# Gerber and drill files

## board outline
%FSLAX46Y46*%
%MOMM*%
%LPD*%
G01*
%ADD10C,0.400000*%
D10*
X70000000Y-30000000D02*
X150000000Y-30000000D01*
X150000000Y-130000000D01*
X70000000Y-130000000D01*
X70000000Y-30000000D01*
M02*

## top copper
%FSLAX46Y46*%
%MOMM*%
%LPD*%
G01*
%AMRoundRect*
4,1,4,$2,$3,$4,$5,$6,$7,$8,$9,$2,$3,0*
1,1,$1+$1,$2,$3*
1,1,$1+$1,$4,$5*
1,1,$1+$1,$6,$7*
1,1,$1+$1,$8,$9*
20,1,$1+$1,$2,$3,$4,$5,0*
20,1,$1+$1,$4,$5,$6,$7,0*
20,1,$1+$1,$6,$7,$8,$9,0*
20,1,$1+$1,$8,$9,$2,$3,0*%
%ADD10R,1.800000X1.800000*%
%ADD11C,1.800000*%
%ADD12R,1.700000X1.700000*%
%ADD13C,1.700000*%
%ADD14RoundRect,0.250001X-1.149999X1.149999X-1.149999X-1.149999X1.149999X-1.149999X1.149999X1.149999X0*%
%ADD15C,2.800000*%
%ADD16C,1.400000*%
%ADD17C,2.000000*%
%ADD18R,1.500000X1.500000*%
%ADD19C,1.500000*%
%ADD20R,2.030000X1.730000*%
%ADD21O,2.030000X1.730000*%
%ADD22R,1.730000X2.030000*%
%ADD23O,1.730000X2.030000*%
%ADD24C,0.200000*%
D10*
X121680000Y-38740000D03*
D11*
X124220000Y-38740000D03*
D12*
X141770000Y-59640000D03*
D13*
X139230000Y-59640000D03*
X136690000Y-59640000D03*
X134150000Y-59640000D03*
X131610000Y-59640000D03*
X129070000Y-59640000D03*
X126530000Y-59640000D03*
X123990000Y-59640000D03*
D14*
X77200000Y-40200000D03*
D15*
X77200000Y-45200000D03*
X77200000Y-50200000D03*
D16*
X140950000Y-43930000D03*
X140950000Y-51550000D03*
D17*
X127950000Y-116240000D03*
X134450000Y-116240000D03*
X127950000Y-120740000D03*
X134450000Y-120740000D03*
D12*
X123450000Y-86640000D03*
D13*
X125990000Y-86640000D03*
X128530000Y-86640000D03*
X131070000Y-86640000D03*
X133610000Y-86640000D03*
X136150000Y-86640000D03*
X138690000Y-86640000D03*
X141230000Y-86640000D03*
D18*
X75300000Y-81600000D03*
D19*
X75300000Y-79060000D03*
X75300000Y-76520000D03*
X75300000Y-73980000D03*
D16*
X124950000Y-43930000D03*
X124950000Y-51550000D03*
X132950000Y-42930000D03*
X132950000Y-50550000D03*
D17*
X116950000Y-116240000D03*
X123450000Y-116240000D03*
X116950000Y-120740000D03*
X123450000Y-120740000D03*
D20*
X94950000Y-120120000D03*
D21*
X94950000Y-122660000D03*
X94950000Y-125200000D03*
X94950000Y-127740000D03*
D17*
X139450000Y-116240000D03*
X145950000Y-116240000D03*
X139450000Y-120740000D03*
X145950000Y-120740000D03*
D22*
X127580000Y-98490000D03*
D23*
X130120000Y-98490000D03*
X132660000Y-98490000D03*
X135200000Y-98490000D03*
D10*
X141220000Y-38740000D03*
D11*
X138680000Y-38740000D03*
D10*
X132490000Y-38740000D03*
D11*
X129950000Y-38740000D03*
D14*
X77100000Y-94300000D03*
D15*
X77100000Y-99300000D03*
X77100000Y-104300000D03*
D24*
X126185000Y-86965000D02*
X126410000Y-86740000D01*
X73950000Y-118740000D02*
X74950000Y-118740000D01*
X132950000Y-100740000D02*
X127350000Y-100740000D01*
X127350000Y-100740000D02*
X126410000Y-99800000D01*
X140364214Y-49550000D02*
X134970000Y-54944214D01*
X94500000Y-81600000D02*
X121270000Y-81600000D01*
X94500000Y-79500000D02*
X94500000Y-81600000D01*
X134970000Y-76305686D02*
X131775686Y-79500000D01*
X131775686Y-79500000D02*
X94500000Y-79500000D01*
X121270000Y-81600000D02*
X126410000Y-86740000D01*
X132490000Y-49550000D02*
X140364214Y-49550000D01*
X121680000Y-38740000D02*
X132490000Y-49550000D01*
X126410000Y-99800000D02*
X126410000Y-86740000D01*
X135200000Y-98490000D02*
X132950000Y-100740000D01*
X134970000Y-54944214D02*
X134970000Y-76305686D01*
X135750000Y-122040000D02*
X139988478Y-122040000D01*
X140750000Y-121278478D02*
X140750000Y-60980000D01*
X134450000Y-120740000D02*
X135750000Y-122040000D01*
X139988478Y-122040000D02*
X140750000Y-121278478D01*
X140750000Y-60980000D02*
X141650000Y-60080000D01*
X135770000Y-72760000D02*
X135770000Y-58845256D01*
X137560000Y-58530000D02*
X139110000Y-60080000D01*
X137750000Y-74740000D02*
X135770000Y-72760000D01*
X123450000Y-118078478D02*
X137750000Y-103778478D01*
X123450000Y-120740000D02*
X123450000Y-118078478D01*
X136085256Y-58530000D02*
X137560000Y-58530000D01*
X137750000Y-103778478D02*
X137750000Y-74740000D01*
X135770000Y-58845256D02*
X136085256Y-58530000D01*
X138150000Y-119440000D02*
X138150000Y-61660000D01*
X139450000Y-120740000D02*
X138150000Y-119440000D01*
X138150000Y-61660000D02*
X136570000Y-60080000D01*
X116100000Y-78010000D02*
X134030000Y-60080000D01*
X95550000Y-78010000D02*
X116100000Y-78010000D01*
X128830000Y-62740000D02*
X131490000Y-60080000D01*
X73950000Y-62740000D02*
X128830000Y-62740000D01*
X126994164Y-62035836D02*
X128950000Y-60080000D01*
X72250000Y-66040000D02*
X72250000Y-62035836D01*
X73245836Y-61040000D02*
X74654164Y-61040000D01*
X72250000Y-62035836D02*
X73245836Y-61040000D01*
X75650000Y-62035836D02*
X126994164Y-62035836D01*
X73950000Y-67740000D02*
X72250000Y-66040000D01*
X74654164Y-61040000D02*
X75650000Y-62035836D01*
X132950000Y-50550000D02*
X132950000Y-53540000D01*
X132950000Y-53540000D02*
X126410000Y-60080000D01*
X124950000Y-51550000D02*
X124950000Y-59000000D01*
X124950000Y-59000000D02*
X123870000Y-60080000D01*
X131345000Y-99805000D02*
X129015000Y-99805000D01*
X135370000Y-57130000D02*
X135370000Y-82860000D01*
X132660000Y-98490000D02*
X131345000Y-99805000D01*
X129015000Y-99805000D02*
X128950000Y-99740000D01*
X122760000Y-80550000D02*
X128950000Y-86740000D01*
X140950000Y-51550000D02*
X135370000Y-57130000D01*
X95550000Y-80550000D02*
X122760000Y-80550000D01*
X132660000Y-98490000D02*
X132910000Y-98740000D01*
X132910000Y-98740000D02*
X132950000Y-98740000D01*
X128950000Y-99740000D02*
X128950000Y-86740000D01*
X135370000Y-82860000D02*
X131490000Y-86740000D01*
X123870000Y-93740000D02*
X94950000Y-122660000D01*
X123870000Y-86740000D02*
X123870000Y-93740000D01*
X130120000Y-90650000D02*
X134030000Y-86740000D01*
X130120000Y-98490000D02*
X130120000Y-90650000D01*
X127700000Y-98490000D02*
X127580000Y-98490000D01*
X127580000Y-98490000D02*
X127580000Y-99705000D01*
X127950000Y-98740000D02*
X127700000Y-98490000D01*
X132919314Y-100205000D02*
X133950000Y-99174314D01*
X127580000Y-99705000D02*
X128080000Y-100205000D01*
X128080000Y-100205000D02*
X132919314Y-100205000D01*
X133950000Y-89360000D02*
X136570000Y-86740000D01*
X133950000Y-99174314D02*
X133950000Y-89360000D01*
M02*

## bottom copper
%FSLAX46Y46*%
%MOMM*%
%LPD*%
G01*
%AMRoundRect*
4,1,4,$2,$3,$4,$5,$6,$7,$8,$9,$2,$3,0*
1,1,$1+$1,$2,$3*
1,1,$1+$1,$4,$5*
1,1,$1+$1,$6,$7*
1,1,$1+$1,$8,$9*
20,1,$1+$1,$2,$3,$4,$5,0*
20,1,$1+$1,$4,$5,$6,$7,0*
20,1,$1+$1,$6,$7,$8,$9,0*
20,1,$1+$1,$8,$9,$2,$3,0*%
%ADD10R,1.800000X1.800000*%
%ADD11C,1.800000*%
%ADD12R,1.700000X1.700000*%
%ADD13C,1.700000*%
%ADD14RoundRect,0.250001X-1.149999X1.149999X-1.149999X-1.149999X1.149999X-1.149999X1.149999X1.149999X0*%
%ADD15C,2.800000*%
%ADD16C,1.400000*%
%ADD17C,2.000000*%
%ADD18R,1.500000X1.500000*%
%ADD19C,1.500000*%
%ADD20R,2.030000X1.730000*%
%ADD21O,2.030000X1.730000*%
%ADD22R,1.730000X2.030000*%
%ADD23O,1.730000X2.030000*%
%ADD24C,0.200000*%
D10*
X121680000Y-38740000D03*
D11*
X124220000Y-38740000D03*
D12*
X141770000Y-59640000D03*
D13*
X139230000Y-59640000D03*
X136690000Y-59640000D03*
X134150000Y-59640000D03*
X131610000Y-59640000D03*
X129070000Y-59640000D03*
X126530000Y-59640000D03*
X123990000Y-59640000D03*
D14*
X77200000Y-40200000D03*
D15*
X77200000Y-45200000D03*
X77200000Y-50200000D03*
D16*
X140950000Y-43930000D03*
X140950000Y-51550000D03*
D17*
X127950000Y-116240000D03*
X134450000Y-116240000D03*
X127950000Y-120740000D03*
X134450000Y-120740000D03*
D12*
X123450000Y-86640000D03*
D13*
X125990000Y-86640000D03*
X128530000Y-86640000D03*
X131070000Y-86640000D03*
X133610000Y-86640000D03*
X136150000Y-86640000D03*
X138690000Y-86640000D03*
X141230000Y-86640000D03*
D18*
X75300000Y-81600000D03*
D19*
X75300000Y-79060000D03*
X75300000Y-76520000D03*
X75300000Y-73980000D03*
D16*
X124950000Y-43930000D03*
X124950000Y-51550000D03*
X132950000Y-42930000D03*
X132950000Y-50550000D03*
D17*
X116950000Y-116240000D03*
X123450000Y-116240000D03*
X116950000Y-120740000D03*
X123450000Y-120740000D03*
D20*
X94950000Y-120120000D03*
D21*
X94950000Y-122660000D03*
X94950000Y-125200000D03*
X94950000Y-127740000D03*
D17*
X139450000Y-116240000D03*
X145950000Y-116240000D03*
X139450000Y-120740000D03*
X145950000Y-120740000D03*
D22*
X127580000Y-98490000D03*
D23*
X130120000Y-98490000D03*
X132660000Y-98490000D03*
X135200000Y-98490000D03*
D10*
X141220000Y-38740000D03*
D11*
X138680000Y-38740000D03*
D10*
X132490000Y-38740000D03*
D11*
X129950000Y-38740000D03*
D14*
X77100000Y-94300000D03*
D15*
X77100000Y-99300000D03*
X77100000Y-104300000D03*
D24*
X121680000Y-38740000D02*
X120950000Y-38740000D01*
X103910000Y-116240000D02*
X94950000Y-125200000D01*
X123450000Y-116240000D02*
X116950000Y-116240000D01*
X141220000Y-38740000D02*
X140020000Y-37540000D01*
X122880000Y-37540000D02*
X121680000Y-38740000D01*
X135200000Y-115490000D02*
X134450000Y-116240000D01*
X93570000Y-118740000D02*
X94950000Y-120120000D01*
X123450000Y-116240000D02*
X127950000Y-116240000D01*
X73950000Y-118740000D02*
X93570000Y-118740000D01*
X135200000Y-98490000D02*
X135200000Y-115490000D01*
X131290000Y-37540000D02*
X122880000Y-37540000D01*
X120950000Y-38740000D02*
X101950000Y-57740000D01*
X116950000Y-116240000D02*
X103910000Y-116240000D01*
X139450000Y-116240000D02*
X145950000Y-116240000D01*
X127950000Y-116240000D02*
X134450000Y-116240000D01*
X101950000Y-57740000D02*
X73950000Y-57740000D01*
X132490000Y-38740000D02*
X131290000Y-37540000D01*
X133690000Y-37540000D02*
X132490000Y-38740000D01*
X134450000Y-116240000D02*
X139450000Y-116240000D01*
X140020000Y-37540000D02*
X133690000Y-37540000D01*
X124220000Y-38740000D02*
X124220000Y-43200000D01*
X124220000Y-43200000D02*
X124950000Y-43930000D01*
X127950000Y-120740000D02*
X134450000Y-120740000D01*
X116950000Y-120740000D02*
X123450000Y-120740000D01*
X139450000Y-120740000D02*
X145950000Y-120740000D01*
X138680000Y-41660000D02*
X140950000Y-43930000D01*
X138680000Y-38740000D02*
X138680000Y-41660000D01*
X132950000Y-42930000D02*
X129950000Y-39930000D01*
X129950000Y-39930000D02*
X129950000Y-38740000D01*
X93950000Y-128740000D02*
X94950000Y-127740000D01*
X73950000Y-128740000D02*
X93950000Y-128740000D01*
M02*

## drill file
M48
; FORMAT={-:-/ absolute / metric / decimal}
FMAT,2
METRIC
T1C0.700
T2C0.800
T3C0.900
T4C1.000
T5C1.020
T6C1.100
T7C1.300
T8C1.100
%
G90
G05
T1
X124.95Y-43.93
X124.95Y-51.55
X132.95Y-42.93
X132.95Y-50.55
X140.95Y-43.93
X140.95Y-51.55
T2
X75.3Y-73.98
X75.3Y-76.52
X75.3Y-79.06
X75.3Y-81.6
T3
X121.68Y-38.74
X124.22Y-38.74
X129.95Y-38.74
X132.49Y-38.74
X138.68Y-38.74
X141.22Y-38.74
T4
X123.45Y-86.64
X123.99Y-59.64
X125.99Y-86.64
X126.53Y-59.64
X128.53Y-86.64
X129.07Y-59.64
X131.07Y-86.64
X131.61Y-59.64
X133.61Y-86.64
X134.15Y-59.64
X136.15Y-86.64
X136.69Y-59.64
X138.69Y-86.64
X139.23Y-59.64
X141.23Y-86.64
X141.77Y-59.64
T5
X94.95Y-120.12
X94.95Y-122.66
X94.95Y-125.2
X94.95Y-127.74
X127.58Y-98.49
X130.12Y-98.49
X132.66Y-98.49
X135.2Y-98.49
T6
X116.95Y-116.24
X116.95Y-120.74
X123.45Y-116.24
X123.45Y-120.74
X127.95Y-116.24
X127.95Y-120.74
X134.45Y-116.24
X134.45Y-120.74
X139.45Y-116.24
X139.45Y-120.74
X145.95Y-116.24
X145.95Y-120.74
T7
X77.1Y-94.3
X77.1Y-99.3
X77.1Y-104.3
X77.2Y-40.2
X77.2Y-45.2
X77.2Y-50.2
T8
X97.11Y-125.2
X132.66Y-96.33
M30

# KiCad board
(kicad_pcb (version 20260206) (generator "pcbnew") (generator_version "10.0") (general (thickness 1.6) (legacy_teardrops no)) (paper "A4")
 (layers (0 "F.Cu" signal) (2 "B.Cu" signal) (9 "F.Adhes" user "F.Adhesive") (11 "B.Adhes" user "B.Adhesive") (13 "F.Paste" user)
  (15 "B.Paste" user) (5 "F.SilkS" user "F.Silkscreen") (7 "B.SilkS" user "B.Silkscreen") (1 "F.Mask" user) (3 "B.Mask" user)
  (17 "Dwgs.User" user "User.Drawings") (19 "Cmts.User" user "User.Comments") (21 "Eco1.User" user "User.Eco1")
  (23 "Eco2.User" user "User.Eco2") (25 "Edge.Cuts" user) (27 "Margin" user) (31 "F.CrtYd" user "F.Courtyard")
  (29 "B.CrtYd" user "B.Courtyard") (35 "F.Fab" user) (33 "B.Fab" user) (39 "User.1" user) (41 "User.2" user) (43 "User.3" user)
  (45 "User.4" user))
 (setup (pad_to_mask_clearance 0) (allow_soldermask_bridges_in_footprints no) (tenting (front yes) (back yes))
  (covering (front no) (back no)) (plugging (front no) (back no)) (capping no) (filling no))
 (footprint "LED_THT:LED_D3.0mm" (layer "F.Cu") (at 121.68 38.74)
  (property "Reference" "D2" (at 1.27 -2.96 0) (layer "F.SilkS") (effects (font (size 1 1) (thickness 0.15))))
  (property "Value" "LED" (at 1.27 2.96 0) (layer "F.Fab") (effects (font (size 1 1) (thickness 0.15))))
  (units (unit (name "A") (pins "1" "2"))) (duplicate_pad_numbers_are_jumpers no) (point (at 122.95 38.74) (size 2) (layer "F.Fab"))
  (pad "1" thru_hole rect (at 0 0) (size 1.8 1.8) (drill 0.9) (layers "*.Cu" "*.Mask") (remove_unused_layers no) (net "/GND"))
  (pad "2" thru_hole circle (at 2.54 0) (size 1.8 1.8) (drill 0.9) (layers "*.Cu" "*.Mask") (remove_unused_layers no) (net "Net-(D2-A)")))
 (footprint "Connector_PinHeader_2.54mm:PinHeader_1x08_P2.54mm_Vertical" (layer "F.Cu") (at 141.77 59.64 -90)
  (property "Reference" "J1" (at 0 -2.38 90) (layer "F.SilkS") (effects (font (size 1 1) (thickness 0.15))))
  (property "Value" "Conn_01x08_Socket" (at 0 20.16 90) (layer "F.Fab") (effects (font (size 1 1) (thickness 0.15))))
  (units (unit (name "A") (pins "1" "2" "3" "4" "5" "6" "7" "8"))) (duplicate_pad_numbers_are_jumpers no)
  (pad "1" thru_hole rect (at 0 0 270) (size 1.7 1.7) (drill 1) (layers "*.Cu" "*.Mask") (remove_unused_layers no) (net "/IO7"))
  (pad "2" thru_hole circle (at 0 2.54 270) (size 1.7 1.7) (drill 1) (layers "*.Cu" "*.Mask") (remove_unused_layers no) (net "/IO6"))
  (pad "3" thru_hole circle (at 0 5.08 270) (size 1.7 1.7) (drill 1) (layers "*.Cu" "*.Mask") (remove_unused_layers no) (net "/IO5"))
  (pad "4" thru_hole circle (at 0 7.62 270) (size 1.7 1.7) (drill 1) (layers "*.Cu" "*.Mask") (remove_unused_layers no) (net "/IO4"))
  (pad "5" thru_hole circle (at 0 10.16 270) (size 1.7 1.7) (drill 1) (layers "*.Cu" "*.Mask") (remove_unused_layers no) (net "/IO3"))
  (pad "6" thru_hole circle (at 0 12.7 270) (size 1.7 1.7) (drill 1) (layers "*.Cu" "*.Mask") (remove_unused_layers no) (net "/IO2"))
  (pad "7" thru_hole circle (at 0 15.24 270) (size 1.7 1.7) (drill 1) (layers "*.Cu" "*.Mask") (remove_unused_layers no) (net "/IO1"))
  (pad "8" thru_hole circle (at 0 17.78 270) (size 1.7 1.7) (drill 1) (layers "*.Cu" "*.Mask") (remove_unused_layers no) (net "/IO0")))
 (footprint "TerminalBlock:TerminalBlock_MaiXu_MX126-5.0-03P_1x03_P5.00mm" (layer "F.Cu") (at 77.2 40.2 -90)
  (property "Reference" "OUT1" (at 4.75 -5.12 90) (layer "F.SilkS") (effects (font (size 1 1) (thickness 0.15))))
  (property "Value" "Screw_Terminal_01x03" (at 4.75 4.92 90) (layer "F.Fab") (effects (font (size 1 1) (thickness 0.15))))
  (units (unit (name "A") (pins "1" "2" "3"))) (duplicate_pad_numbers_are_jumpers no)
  (pad "1" thru_hole roundrect (at 0 0 270) (size 2.8 2.8) (drill 1.3) (layers "*.Cu" "*.Mask") (remove_unused_layers no)
   (roundrect_rratio 0.089286) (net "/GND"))
  (pad "2" thru_hole circle (at 5 0 270) (size 2.8 2.8) (drill 1.3) (layers "*.Cu" "*.Mask") (remove_unused_layers no) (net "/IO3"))
  (pad "3" thru_hole circle (at 10 0 270) (size 2.8 2.8) (drill 1.3) (layers "*.Cu" "*.Mask") (remove_unused_layers no) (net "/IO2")))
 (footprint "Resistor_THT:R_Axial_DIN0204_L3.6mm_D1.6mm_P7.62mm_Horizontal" (layer "F.Cu") (at 140.95 43.93 -90)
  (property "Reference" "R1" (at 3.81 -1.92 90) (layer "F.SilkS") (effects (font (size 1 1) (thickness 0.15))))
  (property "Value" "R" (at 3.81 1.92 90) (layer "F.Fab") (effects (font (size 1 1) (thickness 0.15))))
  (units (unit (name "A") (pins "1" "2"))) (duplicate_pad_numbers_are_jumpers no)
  (pad "1" thru_hole circle (at 0 0 270) (size 1.4 1.4) (drill 0.7) (layers "*.Cu" "*.Mask") (remove_unused_layers no) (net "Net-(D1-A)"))
  (pad "2" thru_hole circle (at 7.62 0 270) (size 1.4 1.4) (drill 0.7) (layers "*.Cu" "*.Mask") (remove_unused_layers no) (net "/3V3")))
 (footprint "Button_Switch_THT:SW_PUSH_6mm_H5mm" (layer "F.Cu") (at 127.95 116.24)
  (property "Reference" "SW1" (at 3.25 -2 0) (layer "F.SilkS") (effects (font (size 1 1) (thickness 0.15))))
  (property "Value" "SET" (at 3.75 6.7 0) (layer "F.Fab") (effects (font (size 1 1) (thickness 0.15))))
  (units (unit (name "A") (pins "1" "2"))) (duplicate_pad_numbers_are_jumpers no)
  (pad "1" thru_hole circle (at 0 0 90) (size 2 2) (drill 1.1) (layers "*.Cu" "*.Mask") (remove_unused_layers no) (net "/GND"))
  (pad "1" thru_hole circle (at 6.5 0 90) (size 2 2) (drill 1.1) (layers "*.Cu" "*.Mask") (remove_unused_layers no) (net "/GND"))
  (pad "2" thru_hole circle (at 0 4.5 90) (size 2 2) (drill 1.1) (layers "*.Cu" "*.Mask") (remove_unused_layers no) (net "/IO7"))
  (pad "2" thru_hole circle (at 6.5 4.5 90) (size 2 2) (drill 1.1) (layers "*.Cu" "*.Mask") (remove_unused_layers no) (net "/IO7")))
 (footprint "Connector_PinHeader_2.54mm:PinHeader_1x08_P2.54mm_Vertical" (layer "F.Cu") (at 123.45 86.64 90)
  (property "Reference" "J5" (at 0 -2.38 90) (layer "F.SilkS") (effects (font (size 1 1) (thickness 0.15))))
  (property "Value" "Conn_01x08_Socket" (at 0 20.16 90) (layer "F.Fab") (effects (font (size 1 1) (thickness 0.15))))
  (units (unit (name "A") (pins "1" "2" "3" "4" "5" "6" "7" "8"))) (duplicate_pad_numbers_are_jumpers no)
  (pad "1" thru_hole rect (at 0 0 90) (size 1.7 1.7) (drill 1) (layers "*.Cu" "*.Mask") (remove_unused_layers no) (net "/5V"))
  (pad "2" thru_hole circle (at 0 2.54 90) (size 1.7 1.7) (drill 1) (layers "*.Cu" "*.Mask") (remove_unused_layers no) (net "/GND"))
  (pad "3" thru_hole circle (at 0 5.08 90) (size 1.7 1.7) (drill 1) (layers "*.Cu" "*.Mask") (remove_unused_layers no) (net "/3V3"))
  (pad "4" thru_hole circle (at 0 7.62 90) (size 1.7 1.7) (drill 1) (layers "*.Cu" "*.Mask") (remove_unused_layers no) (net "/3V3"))
  (pad "5" thru_hole circle (at 0 10.16 90) (size 1.7 1.7) (drill 1) (layers "*.Cu" "*.Mask") (remove_unused_layers no) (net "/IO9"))
  (pad "6" thru_hole circle (at 0 12.7 90) (size 1.7 1.7) (drill 1) (layers "*.Cu" "*.Mask") (remove_unused_layers no) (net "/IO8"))
  (pad "7" thru_hole circle (at 0 15.24 90) (size 1.7 1.7) (drill 1) (layers "*.Cu" "*.Mask") (remove_unused_layers no) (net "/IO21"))
  (pad "8" thru_hole circle (at 0 17.78 90) (size 1.7 1.7) (drill 1) (layers "*.Cu" "*.Mask") (remove_unused_layers no) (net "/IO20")))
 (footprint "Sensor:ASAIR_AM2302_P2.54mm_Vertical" (layer "F.Cu") (at 75.3 81.6 90)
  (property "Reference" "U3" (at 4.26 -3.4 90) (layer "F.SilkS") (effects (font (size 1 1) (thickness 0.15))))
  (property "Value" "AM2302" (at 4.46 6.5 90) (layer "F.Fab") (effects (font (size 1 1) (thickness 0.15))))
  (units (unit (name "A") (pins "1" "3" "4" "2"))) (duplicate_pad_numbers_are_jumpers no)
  (pad "1" thru_hole rect (at 0 0 180) (size 1.5 1.5) (drill 0.8) (layers "*.Cu" "*.Mask") (remove_unused_layers no) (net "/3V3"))
  (pad "2" thru_hole circle (at 2.54 0 180) (size 1.5 1.5) (drill 0.8) (layers "*.Cu" "*.Mask") (remove_unused_layers no) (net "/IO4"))
  (pad "3" thru_hole circle (at 5.08 0 180) (size 1.5 1.5) (drill 0.8) (layers "*.Cu" "*.Mask") (remove_unused_layers no)
   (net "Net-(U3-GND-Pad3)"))
  (pad "4" thru_hole circle (at 7.62 0 180) (size 1.5 1.5) (drill 0.8) (layers "*.Cu" "*.Mask") (remove_unused_layers no)
   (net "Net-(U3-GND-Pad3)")))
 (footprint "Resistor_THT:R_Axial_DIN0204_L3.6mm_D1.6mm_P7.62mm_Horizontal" (layer "F.Cu") (at 124.95 43.93 -90)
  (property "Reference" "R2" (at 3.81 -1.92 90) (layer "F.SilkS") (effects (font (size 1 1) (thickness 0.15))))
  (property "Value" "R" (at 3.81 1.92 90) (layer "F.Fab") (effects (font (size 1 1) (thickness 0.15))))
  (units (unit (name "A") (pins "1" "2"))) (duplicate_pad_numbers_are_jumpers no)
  (pad "1" thru_hole circle (at 0 0 270) (size 1.4 1.4) (drill 0.7) (layers "*.Cu" "*.Mask") (remove_unused_layers no) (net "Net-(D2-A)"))
  (pad "2" thru_hole circle (at 7.62 0 270) (size 1.4 1.4) (drill 0.7) (layers "*.Cu" "*.Mask") (remove_unused_layers no) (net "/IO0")))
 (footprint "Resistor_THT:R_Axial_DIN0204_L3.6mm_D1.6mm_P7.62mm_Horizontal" (layer "F.Cu") (at 132.95 42.93 -90)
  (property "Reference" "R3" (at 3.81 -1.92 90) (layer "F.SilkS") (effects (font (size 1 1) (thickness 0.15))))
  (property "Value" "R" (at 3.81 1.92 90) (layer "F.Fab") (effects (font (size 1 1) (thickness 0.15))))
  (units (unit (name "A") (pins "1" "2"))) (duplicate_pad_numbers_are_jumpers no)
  (pad "1" thru_hole circle (at 0 0 270) (size 1.4 1.4) (drill 0.7) (layers "*.Cu" "*.Mask") (remove_unused_layers no) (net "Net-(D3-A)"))
  (pad "2" thru_hole circle (at 7.62 0 270) (size 1.4 1.4) (drill 0.7) (layers "*.Cu" "*.Mask") (remove_unused_layers no) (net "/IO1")))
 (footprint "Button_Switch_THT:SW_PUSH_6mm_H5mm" (layer "F.Cu") (at 116.95 116.24)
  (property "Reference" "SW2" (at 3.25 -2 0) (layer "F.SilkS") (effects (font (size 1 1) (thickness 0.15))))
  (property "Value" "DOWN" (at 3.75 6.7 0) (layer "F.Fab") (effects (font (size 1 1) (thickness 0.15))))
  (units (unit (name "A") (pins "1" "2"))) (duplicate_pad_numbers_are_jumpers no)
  (pad "1" thru_hole circle (at 0 0 90) (size 2 2) (drill 1.1) (layers "*.Cu" "*.Mask") (remove_unused_layers no) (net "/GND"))
  (pad "1" thru_hole circle (at 6.5 0 90) (size 2 2) (drill 1.1) (layers "*.Cu" "*.Mask") (remove_unused_layers no) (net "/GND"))
  (pad "2" thru_hole circle (at 0 4.5 90) (size 2 2) (drill 1.1) (layers "*.Cu" "*.Mask") (remove_unused_layers no) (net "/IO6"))
  (pad "2" thru_hole circle (at 6.5 4.5 90) (size 2 2) (drill 1.1) (layers "*.Cu" "*.Mask") (remove_unused_layers no) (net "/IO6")))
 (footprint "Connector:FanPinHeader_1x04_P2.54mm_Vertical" (layer "F.Cu") (at 94.95 120.12 -90)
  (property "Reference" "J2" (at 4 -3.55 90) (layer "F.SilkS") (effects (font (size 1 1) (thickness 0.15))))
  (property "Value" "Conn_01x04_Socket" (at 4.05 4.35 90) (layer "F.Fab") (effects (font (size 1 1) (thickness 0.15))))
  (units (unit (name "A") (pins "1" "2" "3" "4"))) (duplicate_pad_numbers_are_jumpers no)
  (pad "" np_thru_hole circle (at 5.08 -2.16) (size 1.1 1.1) (drill 1.1) (layers "*.Cu" "*.Mask"))
  (pad "1" thru_hole rect (at 0 0) (size 2.03 1.73) (drill 1.02) (layers "*.Cu" "*.Mask") (remove_unused_layers no) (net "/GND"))
  (pad "2" thru_hole oval (at 2.54 0) (size 2.03 1.73) (drill 1.02) (layers "*.Cu" "*.Mask") (remove_unused_layers no) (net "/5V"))
  (pad "3" thru_hole oval (at 5.08 0) (size 2.03 1.73) (drill 1.02) (layers "*.Cu" "*.Mask") (remove_unused_layers no) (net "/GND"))
  (pad "4" thru_hole oval (at 7.62 0) (size 2.03 1.73) (drill 1.02) (layers "*.Cu" "*.Mask") (remove_unused_layers no) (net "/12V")))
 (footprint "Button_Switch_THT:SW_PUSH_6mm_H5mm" (layer "F.Cu") (at 139.45 116.24)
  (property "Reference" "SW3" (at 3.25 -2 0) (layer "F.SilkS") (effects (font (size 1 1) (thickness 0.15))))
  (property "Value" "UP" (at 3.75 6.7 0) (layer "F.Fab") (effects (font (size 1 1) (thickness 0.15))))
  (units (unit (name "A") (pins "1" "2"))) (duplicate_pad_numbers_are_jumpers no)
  (pad "1" thru_hole circle (at 0 0 90) (size 2 2) (drill 1.1) (layers "*.Cu" "*.Mask") (remove_unused_layers no) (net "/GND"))
  (pad "1" thru_hole circle (at 6.5 0 90) (size 2 2) (drill 1.1) (layers "*.Cu" "*.Mask") (remove_unused_layers no) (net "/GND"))
  (pad "2" thru_hole circle (at 0 4.5 90) (size 2 2) (drill 1.1) (layers "*.Cu" "*.Mask") (remove_unused_layers no) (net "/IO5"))
  (pad "2" thru_hole circle (at 6.5 4.5 90) (size 2 2) (drill 1.1) (layers "*.Cu" "*.Mask") (remove_unused_layers no) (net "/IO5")))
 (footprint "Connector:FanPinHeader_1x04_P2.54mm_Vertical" (layer "F.Cu") (at 127.58 98.49)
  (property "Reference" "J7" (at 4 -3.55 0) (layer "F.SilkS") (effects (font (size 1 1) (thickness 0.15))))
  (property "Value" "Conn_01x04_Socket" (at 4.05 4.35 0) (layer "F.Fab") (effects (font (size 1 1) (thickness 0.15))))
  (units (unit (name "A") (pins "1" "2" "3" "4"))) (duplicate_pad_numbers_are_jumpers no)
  (pad "" np_thru_hole circle (at 5.08 -2.16 90) (size 1.1 1.1) (drill 1.1) (layers "*.Cu" "*.Mask"))
  (pad "1" thru_hole rect (at 0 0 90) (size 2.03 1.73) (drill 1.02) (layers "*.Cu" "*.Mask") (remove_unused_layers no) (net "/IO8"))
  (pad "2" thru_hole oval (at 2.54 0 90) (size 2.03 1.73) (drill 1.02) (layers "*.Cu" "*.Mask") (remove_unused_layers no) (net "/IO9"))
  (pad "3" thru_hole oval (at 5.08 0 90) (size 2.03 1.73) (drill 1.02) (layers "*.Cu" "*.Mask") (remove_unused_layers no) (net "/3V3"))
  (pad "4" thru_hole oval (at 7.62 0 90) (size 2.03 1.73) (drill 1.02) (layers "*.Cu" "*.Mask") (remove_unused_layers no) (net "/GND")))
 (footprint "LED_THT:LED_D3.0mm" (layer "F.Cu") (at 141.22 38.74 180)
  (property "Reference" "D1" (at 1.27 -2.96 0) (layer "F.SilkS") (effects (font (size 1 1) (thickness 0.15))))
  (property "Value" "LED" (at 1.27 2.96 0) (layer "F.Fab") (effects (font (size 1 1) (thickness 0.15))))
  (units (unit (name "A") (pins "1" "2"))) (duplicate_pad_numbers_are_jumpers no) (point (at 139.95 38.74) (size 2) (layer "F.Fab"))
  (pad "1" thru_hole rect (at 0 0 180) (size 1.8 1.8) (drill 0.9) (layers "*.Cu" "*.Mask") (remove_unused_layers no) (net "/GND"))
  (pad "2" thru_hole circle (at 2.54 0 180) (size 1.8 1.8) (drill 0.9) (layers "*.Cu" "*.Mask") (remove_unused_layers no) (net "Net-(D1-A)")))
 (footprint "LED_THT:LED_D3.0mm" (layer "F.Cu") (at 132.49 38.74 180)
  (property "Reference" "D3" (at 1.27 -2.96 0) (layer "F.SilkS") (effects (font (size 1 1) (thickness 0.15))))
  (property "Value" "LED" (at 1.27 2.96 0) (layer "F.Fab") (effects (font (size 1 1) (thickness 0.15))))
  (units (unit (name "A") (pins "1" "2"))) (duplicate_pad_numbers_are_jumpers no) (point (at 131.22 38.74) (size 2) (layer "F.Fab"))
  (pad "1" thru_hole rect (at 0 0 180) (size 1.8 1.8) (drill 0.9) (layers "*.Cu" "*.Mask") (remove_unused_layers no) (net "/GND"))
  (pad "2" thru_hole circle (at 2.54 0 180) (size 1.8 1.8) (drill 0.9) (layers "*.Cu" "*.Mask") (remove_unused_layers no) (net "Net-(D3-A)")))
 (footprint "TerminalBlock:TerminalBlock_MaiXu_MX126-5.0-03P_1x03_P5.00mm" (layer "F.Cu") (at 77.1 94.3 -90)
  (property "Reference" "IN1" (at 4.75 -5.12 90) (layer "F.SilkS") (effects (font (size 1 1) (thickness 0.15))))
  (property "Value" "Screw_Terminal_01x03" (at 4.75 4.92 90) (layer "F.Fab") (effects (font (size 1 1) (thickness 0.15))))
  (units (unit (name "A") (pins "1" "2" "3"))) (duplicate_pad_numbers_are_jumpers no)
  (pad "1" thru_hole roundrect (at 0 0 270) (size 2.8 2.8) (drill 1.3) (layers "*.Cu" "*.Mask") (remove_unused_layers no)
   (roundrect_rratio 0.089286) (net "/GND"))
  (pad "2" thru_hole circle (at 5 0 270) (size 2.8 2.8) (drill 1.3) (layers "*.Cu" "*.Mask") (remove_unused_layers no)
   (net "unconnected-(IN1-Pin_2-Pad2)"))
  (pad "3" thru_hole circle (at 10 0 270) (size 2.8 2.8) (drill 1.3) (layers "*.Cu" "*.Mask") (remove_unused_layers no) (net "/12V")))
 (gr_rect (start 70 30) (end 150 130) (stroke (width 0.4) (type solid)) (fill no) (locked yes) (layer "Edge.Cuts"))
 (segment (start 126.185 86.965) (end 126.41 86.74) (width 0.2) (layer "F.Cu") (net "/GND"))
 (segment (start 73.95 118.74) (end 74.95 118.74) (width 0.2) (layer "F.Cu") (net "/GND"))
 (segment (start 132.95 100.74) (end 127.35 100.74) (width 0.2) (layer "F.Cu") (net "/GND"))
 (segment (start 127.35 100.74) (end 126.41 99.8) (width 0.2) (layer "F.Cu") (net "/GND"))
 (segment (start 140.364214 49.55) (end 134.97 54.944214) (width 0.2) (layer "F.Cu") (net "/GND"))
 (segment (start 94.5 81.6) (end 121.27 81.6) (width 0.2) (layer "F.Cu") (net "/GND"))
 (segment (start 94.5 79.5) (end 94.5 81.6) (width 0.2) (layer "F.Cu") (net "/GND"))
 (segment (start 134.97 76.305686) (end 131.775686 79.5) (width 0.2) (layer "F.Cu") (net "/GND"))
 (segment (start 131.775686 79.5) (end 94.5 79.5) (width 0.2) (layer "F.Cu") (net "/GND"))
 (segment (start 121.27 81.6) (end 126.41 86.74) (width 0.2) (layer "F.Cu") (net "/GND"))
 (segment (start 132.49 49.55) (end 140.364214 49.55) (width 0.2) (layer "F.Cu") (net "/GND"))
 (segment (start 121.68 38.74) (end 132.49 49.55) (width 0.2) (layer "F.Cu") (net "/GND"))
 (segment (start 126.41 99.8) (end 126.41 86.74) (width 0.2) (layer "F.Cu") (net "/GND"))
 (segment (start 135.2 98.49) (end 132.95 100.74) (width 0.2) (layer "F.Cu") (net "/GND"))
 (segment (start 134.97 54.944214) (end 134.97 76.305686) (width 0.2) (layer "F.Cu") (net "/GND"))
 (segment (start 121.68 38.74) (end 120.95 38.74) (width 0.2) (layer "B.Cu") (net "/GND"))
 (segment (start 103.91 116.24) (end 94.95 125.2) (width 0.2) (layer "B.Cu") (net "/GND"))
 (segment (start 123.45 116.24) (end 116.95 116.24) (width 0.2) (layer "B.Cu") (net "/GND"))
 (segment (start 141.22 38.74) (end 140.02 37.54) (width 0.2) (layer "B.Cu") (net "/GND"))
 (segment (start 122.88 37.54) (end 121.68 38.74) (width 0.2) (layer "B.Cu") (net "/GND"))
 (segment (start 135.2 115.49) (end 134.45 116.24) (width 0.2) (layer "B.Cu") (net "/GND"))
 (segment (start 93.57 118.74) (end 94.95 120.12) (width 0.2) (layer "B.Cu") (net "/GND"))
 (segment (start 123.45 116.24) (end 127.95 116.24) (width 0.2) (layer "B.Cu") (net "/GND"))
 (segment (start 73.95 118.74) (end 93.57 118.74) (width 0.2) (layer "B.Cu") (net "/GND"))
 (segment (start 135.2 98.49) (end 135.2 115.49) (width 0.2) (layer "B.Cu") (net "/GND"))
 (segment (start 131.29 37.54) (end 122.88 37.54) (width 0.2) (layer "B.Cu") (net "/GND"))
 (segment (start 120.95 38.74) (end 101.95 57.74) (width 0.2) (layer "B.Cu") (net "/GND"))
 (segment (start 116.95 116.24) (end 103.91 116.24) (width 0.2) (layer "B.Cu") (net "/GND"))
 (segment (start 139.45 116.24) (end 145.95 116.24) (width 0.2) (layer "B.Cu") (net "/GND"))
 (segment (start 127.95 116.24) (end 134.45 116.24) (width 0.2) (layer "B.Cu") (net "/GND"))
 (segment (start 101.95 57.74) (end 73.95 57.74) (width 0.2) (layer "B.Cu") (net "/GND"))
 (segment (start 132.49 38.74) (end 131.29 37.54) (width 0.2) (layer "B.Cu") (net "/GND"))
 (segment (start 133.69 37.54) (end 132.49 38.74) (width 0.2) (layer "B.Cu") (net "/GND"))
 (segment (start 134.45 116.24) (end 139.45 116.24) (width 0.2) (layer "B.Cu") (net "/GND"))
 (segment (start 140.02 37.54) (end 133.69 37.54) (width 0.2) (layer "B.Cu") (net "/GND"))
 (segment (start 124.22 38.74) (end 124.22 43.2) (width 0.2) (layer "B.Cu") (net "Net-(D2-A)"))
 (segment (start 124.22 43.2) (end 124.95 43.93) (width 0.2) (layer "B.Cu") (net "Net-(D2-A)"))
 (segment (start 135.75 122.04) (end 139.988478 122.04) (width 0.2) (layer "F.Cu") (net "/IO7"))
 (segment (start 140.75 121.278478) (end 140.75 60.98) (width 0.2) (layer "F.Cu") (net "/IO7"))
 (segment (start 134.45 120.74) (end 135.75 122.04) (width 0.2) (layer "F.Cu") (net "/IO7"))
 (segment (start 139.988478 122.04) (end 140.75 121.278478) (width 0.2) (layer "F.Cu") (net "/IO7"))
 (segment (start 140.75 60.98) (end 141.65 60.08) (width 0.2) (layer "F.Cu") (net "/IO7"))
 (segment (start 127.95 120.74) (end 134.45 120.74) (width 0.2) (layer "B.Cu") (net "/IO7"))
 (segment (start 135.77 72.76) (end 135.77 58.845256) (width 0.2) (layer "F.Cu") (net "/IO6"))
 (segment (start 137.56 58.53) (end 139.11 60.08) (width 0.2) (layer "F.Cu") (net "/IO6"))
 (segment (start 137.75 74.74) (end 135.77 72.76) (width 0.2) (layer "F.Cu") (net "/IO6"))
 (segment (start 123.45 118.078478) (end 137.75 103.778478) (width 0.2) (layer "F.Cu") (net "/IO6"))
 (segment (start 123.45 120.74) (end 123.45 118.078478) (width 0.2) (layer "F.Cu") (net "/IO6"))
 (segment (start 136.085256 58.53) (end 137.56 58.53) (width 0.2) (layer "F.Cu") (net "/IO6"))
 (segment (start 137.75 103.778478) (end 137.75 74.74) (width 0.2) (layer "F.Cu") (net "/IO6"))
 (segment (start 135.77 58.845256) (end 136.085256 58.53) (width 0.2) (layer "F.Cu") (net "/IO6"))
 (segment (start 116.95 120.74) (end 123.45 120.74) (width 0.2) (layer "B.Cu") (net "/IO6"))
 (segment (start 138.15 119.44) (end 138.15 61.66) (width 0.2) (layer "F.Cu") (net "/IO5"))
 (segment (start 139.45 120.74) (end 138.15 119.44) (width 0.2) (layer "F.Cu") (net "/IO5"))
 (segment (start 138.15 61.66) (end 136.57 60.08) (width 0.2) (layer "F.Cu") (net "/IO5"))
 (segment (start 139.45 120.74) (end 145.95 120.74) (width 0.2) (layer "B.Cu") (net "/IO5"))
 (segment (start 116.1 78.01) (end 134.03 60.08) (width 0.2) (layer "F.Cu") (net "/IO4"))
 (segment (start 95.55 78.01) (end 116.1 78.01) (width 0.2) (layer "F.Cu") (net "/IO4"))
 (segment (start 128.83 62.74) (end 131.49 60.08) (width 0.2) (layer "F.Cu") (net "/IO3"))
 (segment (start 73.95 62.74) (end 128.83 62.74) (width 0.2) (layer "F.Cu") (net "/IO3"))
 (segment (start 126.994164 62.035836) (end 128.95 60.08) (width 0.2) (layer "F.Cu") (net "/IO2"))
 (segment (start 72.25 66.04) (end 72.25 62.035836) (width 0.2) (layer "F.Cu") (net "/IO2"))
 (segment (start 73.245836 61.04) (end 74.654164 61.04) (width 0.2) (layer "F.Cu") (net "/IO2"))
 (segment (start 72.25 62.035836) (end 73.245836 61.04) (width 0.2) (layer "F.Cu") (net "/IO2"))
 (segment (start 75.65 62.035836) (end 126.994164 62.035836) (width 0.2) (layer "F.Cu") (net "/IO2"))
 (segment (start 73.95 67.74) (end 72.25 66.04) (width 0.2) (layer "F.Cu") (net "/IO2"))
 (segment (start 74.654164 61.04) (end 75.65 62.035836) (width 0.2) (layer "F.Cu") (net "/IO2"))
 (segment (start 132.95 50.55) (end 132.95 53.54) (width 0.2) (layer "F.Cu") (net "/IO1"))
 (segment (start 132.95 53.54) (end 126.41 60.08) (width 0.2) (layer "F.Cu") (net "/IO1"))
 (segment (start 124.95 51.55) (end 124.95 59) (width 0.2) (layer "F.Cu") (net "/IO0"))
 (segment (start 124.95 59) (end 123.87 60.08) (width 0.2) (layer "F.Cu") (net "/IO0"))
 (segment (start 138.68 41.66) (end 140.95 43.93) (width 0.2) (layer "B.Cu") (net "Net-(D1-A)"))
 (segment (start 138.68 38.74) (end 138.68 41.66) (width 0.2) (layer "B.Cu") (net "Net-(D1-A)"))
 (segment (start 131.345 99.805) (end 129.015 99.805) (width 0.2) (layer "F.Cu") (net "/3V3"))
 (segment (start 135.37 57.13) (end 135.37 82.86) (width 0.2) (layer "F.Cu") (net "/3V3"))
 (segment (start 132.66 98.49) (end 131.345 99.805) (width 0.2) (layer "F.Cu") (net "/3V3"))
 (segment (start 129.015 99.805) (end 128.95 99.74) (width 0.2) (layer "F.Cu") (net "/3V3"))
 (segment (start 122.76 80.55) (end 128.95 86.74) (width 0.2) (layer "F.Cu") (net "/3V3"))
 (segment (start 140.95 51.55) (end 135.37 57.13) (width 0.2) (layer "F.Cu") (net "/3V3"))
 (segment (start 95.55 80.55) (end 122.76 80.55) (width 0.2) (layer "F.Cu") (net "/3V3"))
 (segment (start 132.66 98.49) (end 132.91 98.74) (width 0.2) (layer "F.Cu") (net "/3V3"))
 (segment (start 132.91 98.74) (end 132.95 98.74) (width 0.2) (layer "F.Cu") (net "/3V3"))
 (segment (start 128.95 99.74) (end 128.95 86.74) (width 0.2) (layer "F.Cu") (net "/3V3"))
 (segment (start 135.37 82.86) (end 131.49 86.74) (width 0.2) (layer "F.Cu") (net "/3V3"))
 (segment (start 123.87 93.74) (end 94.95 122.66) (width 0.2) (layer "F.Cu") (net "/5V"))
 (segment (start 123.87 86.74) (end 123.87 93.74) (width 0.2) (layer "F.Cu") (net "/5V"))
 (segment (start 130.12 90.65) (end 134.03 86.74) (width 0.2) (layer "F.Cu") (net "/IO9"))
 (segment (start 130.12 98.49) (end 130.12 90.65) (width 0.2) (layer "F.Cu") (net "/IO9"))
 (segment (start 127.7 98.49) (end 127.58 98.49) (width 0.2) (layer "F.Cu") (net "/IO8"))
 (segment (start 127.58 98.49) (end 127.58 99.705) (width 0.2) (layer "F.Cu") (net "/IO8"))
 (segment (start 127.95 98.74) (end 127.7 98.49) (width 0.2) (layer "F.Cu") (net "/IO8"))
 (segment (start 132.919314 100.205) (end 133.95 99.174314) (width 0.2) (layer "F.Cu") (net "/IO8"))
 (segment (start 127.58 99.705) (end 128.08 100.205) (width 0.2) (layer "F.Cu") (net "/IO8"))
 (segment (start 128.08 100.205) (end 132.919314 100.205) (width 0.2) (layer "F.Cu") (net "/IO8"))
 (segment (start 133.95 89.36) (end 136.57 86.74) (width 0.2) (layer "F.Cu") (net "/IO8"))
 (segment (start 133.95 99.174314) (end 133.95 89.36) (width 0.2) (layer "F.Cu") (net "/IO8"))
 (segment (start 132.95 42.93) (end 129.95 39.93) (width 0.2) (layer "B.Cu") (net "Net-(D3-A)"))
 (segment (start 129.95 39.93) (end 129.95 38.74) (width 0.2) (layer "B.Cu") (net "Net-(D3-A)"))
 (segment (start 93.95 128.74) (end 94.95 127.74) (width 0.2) (layer "B.Cu") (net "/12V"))
 (segment (start 73.95 128.74) (end 93.95 128.74) (width 0.2) (layer "B.Cu") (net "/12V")))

